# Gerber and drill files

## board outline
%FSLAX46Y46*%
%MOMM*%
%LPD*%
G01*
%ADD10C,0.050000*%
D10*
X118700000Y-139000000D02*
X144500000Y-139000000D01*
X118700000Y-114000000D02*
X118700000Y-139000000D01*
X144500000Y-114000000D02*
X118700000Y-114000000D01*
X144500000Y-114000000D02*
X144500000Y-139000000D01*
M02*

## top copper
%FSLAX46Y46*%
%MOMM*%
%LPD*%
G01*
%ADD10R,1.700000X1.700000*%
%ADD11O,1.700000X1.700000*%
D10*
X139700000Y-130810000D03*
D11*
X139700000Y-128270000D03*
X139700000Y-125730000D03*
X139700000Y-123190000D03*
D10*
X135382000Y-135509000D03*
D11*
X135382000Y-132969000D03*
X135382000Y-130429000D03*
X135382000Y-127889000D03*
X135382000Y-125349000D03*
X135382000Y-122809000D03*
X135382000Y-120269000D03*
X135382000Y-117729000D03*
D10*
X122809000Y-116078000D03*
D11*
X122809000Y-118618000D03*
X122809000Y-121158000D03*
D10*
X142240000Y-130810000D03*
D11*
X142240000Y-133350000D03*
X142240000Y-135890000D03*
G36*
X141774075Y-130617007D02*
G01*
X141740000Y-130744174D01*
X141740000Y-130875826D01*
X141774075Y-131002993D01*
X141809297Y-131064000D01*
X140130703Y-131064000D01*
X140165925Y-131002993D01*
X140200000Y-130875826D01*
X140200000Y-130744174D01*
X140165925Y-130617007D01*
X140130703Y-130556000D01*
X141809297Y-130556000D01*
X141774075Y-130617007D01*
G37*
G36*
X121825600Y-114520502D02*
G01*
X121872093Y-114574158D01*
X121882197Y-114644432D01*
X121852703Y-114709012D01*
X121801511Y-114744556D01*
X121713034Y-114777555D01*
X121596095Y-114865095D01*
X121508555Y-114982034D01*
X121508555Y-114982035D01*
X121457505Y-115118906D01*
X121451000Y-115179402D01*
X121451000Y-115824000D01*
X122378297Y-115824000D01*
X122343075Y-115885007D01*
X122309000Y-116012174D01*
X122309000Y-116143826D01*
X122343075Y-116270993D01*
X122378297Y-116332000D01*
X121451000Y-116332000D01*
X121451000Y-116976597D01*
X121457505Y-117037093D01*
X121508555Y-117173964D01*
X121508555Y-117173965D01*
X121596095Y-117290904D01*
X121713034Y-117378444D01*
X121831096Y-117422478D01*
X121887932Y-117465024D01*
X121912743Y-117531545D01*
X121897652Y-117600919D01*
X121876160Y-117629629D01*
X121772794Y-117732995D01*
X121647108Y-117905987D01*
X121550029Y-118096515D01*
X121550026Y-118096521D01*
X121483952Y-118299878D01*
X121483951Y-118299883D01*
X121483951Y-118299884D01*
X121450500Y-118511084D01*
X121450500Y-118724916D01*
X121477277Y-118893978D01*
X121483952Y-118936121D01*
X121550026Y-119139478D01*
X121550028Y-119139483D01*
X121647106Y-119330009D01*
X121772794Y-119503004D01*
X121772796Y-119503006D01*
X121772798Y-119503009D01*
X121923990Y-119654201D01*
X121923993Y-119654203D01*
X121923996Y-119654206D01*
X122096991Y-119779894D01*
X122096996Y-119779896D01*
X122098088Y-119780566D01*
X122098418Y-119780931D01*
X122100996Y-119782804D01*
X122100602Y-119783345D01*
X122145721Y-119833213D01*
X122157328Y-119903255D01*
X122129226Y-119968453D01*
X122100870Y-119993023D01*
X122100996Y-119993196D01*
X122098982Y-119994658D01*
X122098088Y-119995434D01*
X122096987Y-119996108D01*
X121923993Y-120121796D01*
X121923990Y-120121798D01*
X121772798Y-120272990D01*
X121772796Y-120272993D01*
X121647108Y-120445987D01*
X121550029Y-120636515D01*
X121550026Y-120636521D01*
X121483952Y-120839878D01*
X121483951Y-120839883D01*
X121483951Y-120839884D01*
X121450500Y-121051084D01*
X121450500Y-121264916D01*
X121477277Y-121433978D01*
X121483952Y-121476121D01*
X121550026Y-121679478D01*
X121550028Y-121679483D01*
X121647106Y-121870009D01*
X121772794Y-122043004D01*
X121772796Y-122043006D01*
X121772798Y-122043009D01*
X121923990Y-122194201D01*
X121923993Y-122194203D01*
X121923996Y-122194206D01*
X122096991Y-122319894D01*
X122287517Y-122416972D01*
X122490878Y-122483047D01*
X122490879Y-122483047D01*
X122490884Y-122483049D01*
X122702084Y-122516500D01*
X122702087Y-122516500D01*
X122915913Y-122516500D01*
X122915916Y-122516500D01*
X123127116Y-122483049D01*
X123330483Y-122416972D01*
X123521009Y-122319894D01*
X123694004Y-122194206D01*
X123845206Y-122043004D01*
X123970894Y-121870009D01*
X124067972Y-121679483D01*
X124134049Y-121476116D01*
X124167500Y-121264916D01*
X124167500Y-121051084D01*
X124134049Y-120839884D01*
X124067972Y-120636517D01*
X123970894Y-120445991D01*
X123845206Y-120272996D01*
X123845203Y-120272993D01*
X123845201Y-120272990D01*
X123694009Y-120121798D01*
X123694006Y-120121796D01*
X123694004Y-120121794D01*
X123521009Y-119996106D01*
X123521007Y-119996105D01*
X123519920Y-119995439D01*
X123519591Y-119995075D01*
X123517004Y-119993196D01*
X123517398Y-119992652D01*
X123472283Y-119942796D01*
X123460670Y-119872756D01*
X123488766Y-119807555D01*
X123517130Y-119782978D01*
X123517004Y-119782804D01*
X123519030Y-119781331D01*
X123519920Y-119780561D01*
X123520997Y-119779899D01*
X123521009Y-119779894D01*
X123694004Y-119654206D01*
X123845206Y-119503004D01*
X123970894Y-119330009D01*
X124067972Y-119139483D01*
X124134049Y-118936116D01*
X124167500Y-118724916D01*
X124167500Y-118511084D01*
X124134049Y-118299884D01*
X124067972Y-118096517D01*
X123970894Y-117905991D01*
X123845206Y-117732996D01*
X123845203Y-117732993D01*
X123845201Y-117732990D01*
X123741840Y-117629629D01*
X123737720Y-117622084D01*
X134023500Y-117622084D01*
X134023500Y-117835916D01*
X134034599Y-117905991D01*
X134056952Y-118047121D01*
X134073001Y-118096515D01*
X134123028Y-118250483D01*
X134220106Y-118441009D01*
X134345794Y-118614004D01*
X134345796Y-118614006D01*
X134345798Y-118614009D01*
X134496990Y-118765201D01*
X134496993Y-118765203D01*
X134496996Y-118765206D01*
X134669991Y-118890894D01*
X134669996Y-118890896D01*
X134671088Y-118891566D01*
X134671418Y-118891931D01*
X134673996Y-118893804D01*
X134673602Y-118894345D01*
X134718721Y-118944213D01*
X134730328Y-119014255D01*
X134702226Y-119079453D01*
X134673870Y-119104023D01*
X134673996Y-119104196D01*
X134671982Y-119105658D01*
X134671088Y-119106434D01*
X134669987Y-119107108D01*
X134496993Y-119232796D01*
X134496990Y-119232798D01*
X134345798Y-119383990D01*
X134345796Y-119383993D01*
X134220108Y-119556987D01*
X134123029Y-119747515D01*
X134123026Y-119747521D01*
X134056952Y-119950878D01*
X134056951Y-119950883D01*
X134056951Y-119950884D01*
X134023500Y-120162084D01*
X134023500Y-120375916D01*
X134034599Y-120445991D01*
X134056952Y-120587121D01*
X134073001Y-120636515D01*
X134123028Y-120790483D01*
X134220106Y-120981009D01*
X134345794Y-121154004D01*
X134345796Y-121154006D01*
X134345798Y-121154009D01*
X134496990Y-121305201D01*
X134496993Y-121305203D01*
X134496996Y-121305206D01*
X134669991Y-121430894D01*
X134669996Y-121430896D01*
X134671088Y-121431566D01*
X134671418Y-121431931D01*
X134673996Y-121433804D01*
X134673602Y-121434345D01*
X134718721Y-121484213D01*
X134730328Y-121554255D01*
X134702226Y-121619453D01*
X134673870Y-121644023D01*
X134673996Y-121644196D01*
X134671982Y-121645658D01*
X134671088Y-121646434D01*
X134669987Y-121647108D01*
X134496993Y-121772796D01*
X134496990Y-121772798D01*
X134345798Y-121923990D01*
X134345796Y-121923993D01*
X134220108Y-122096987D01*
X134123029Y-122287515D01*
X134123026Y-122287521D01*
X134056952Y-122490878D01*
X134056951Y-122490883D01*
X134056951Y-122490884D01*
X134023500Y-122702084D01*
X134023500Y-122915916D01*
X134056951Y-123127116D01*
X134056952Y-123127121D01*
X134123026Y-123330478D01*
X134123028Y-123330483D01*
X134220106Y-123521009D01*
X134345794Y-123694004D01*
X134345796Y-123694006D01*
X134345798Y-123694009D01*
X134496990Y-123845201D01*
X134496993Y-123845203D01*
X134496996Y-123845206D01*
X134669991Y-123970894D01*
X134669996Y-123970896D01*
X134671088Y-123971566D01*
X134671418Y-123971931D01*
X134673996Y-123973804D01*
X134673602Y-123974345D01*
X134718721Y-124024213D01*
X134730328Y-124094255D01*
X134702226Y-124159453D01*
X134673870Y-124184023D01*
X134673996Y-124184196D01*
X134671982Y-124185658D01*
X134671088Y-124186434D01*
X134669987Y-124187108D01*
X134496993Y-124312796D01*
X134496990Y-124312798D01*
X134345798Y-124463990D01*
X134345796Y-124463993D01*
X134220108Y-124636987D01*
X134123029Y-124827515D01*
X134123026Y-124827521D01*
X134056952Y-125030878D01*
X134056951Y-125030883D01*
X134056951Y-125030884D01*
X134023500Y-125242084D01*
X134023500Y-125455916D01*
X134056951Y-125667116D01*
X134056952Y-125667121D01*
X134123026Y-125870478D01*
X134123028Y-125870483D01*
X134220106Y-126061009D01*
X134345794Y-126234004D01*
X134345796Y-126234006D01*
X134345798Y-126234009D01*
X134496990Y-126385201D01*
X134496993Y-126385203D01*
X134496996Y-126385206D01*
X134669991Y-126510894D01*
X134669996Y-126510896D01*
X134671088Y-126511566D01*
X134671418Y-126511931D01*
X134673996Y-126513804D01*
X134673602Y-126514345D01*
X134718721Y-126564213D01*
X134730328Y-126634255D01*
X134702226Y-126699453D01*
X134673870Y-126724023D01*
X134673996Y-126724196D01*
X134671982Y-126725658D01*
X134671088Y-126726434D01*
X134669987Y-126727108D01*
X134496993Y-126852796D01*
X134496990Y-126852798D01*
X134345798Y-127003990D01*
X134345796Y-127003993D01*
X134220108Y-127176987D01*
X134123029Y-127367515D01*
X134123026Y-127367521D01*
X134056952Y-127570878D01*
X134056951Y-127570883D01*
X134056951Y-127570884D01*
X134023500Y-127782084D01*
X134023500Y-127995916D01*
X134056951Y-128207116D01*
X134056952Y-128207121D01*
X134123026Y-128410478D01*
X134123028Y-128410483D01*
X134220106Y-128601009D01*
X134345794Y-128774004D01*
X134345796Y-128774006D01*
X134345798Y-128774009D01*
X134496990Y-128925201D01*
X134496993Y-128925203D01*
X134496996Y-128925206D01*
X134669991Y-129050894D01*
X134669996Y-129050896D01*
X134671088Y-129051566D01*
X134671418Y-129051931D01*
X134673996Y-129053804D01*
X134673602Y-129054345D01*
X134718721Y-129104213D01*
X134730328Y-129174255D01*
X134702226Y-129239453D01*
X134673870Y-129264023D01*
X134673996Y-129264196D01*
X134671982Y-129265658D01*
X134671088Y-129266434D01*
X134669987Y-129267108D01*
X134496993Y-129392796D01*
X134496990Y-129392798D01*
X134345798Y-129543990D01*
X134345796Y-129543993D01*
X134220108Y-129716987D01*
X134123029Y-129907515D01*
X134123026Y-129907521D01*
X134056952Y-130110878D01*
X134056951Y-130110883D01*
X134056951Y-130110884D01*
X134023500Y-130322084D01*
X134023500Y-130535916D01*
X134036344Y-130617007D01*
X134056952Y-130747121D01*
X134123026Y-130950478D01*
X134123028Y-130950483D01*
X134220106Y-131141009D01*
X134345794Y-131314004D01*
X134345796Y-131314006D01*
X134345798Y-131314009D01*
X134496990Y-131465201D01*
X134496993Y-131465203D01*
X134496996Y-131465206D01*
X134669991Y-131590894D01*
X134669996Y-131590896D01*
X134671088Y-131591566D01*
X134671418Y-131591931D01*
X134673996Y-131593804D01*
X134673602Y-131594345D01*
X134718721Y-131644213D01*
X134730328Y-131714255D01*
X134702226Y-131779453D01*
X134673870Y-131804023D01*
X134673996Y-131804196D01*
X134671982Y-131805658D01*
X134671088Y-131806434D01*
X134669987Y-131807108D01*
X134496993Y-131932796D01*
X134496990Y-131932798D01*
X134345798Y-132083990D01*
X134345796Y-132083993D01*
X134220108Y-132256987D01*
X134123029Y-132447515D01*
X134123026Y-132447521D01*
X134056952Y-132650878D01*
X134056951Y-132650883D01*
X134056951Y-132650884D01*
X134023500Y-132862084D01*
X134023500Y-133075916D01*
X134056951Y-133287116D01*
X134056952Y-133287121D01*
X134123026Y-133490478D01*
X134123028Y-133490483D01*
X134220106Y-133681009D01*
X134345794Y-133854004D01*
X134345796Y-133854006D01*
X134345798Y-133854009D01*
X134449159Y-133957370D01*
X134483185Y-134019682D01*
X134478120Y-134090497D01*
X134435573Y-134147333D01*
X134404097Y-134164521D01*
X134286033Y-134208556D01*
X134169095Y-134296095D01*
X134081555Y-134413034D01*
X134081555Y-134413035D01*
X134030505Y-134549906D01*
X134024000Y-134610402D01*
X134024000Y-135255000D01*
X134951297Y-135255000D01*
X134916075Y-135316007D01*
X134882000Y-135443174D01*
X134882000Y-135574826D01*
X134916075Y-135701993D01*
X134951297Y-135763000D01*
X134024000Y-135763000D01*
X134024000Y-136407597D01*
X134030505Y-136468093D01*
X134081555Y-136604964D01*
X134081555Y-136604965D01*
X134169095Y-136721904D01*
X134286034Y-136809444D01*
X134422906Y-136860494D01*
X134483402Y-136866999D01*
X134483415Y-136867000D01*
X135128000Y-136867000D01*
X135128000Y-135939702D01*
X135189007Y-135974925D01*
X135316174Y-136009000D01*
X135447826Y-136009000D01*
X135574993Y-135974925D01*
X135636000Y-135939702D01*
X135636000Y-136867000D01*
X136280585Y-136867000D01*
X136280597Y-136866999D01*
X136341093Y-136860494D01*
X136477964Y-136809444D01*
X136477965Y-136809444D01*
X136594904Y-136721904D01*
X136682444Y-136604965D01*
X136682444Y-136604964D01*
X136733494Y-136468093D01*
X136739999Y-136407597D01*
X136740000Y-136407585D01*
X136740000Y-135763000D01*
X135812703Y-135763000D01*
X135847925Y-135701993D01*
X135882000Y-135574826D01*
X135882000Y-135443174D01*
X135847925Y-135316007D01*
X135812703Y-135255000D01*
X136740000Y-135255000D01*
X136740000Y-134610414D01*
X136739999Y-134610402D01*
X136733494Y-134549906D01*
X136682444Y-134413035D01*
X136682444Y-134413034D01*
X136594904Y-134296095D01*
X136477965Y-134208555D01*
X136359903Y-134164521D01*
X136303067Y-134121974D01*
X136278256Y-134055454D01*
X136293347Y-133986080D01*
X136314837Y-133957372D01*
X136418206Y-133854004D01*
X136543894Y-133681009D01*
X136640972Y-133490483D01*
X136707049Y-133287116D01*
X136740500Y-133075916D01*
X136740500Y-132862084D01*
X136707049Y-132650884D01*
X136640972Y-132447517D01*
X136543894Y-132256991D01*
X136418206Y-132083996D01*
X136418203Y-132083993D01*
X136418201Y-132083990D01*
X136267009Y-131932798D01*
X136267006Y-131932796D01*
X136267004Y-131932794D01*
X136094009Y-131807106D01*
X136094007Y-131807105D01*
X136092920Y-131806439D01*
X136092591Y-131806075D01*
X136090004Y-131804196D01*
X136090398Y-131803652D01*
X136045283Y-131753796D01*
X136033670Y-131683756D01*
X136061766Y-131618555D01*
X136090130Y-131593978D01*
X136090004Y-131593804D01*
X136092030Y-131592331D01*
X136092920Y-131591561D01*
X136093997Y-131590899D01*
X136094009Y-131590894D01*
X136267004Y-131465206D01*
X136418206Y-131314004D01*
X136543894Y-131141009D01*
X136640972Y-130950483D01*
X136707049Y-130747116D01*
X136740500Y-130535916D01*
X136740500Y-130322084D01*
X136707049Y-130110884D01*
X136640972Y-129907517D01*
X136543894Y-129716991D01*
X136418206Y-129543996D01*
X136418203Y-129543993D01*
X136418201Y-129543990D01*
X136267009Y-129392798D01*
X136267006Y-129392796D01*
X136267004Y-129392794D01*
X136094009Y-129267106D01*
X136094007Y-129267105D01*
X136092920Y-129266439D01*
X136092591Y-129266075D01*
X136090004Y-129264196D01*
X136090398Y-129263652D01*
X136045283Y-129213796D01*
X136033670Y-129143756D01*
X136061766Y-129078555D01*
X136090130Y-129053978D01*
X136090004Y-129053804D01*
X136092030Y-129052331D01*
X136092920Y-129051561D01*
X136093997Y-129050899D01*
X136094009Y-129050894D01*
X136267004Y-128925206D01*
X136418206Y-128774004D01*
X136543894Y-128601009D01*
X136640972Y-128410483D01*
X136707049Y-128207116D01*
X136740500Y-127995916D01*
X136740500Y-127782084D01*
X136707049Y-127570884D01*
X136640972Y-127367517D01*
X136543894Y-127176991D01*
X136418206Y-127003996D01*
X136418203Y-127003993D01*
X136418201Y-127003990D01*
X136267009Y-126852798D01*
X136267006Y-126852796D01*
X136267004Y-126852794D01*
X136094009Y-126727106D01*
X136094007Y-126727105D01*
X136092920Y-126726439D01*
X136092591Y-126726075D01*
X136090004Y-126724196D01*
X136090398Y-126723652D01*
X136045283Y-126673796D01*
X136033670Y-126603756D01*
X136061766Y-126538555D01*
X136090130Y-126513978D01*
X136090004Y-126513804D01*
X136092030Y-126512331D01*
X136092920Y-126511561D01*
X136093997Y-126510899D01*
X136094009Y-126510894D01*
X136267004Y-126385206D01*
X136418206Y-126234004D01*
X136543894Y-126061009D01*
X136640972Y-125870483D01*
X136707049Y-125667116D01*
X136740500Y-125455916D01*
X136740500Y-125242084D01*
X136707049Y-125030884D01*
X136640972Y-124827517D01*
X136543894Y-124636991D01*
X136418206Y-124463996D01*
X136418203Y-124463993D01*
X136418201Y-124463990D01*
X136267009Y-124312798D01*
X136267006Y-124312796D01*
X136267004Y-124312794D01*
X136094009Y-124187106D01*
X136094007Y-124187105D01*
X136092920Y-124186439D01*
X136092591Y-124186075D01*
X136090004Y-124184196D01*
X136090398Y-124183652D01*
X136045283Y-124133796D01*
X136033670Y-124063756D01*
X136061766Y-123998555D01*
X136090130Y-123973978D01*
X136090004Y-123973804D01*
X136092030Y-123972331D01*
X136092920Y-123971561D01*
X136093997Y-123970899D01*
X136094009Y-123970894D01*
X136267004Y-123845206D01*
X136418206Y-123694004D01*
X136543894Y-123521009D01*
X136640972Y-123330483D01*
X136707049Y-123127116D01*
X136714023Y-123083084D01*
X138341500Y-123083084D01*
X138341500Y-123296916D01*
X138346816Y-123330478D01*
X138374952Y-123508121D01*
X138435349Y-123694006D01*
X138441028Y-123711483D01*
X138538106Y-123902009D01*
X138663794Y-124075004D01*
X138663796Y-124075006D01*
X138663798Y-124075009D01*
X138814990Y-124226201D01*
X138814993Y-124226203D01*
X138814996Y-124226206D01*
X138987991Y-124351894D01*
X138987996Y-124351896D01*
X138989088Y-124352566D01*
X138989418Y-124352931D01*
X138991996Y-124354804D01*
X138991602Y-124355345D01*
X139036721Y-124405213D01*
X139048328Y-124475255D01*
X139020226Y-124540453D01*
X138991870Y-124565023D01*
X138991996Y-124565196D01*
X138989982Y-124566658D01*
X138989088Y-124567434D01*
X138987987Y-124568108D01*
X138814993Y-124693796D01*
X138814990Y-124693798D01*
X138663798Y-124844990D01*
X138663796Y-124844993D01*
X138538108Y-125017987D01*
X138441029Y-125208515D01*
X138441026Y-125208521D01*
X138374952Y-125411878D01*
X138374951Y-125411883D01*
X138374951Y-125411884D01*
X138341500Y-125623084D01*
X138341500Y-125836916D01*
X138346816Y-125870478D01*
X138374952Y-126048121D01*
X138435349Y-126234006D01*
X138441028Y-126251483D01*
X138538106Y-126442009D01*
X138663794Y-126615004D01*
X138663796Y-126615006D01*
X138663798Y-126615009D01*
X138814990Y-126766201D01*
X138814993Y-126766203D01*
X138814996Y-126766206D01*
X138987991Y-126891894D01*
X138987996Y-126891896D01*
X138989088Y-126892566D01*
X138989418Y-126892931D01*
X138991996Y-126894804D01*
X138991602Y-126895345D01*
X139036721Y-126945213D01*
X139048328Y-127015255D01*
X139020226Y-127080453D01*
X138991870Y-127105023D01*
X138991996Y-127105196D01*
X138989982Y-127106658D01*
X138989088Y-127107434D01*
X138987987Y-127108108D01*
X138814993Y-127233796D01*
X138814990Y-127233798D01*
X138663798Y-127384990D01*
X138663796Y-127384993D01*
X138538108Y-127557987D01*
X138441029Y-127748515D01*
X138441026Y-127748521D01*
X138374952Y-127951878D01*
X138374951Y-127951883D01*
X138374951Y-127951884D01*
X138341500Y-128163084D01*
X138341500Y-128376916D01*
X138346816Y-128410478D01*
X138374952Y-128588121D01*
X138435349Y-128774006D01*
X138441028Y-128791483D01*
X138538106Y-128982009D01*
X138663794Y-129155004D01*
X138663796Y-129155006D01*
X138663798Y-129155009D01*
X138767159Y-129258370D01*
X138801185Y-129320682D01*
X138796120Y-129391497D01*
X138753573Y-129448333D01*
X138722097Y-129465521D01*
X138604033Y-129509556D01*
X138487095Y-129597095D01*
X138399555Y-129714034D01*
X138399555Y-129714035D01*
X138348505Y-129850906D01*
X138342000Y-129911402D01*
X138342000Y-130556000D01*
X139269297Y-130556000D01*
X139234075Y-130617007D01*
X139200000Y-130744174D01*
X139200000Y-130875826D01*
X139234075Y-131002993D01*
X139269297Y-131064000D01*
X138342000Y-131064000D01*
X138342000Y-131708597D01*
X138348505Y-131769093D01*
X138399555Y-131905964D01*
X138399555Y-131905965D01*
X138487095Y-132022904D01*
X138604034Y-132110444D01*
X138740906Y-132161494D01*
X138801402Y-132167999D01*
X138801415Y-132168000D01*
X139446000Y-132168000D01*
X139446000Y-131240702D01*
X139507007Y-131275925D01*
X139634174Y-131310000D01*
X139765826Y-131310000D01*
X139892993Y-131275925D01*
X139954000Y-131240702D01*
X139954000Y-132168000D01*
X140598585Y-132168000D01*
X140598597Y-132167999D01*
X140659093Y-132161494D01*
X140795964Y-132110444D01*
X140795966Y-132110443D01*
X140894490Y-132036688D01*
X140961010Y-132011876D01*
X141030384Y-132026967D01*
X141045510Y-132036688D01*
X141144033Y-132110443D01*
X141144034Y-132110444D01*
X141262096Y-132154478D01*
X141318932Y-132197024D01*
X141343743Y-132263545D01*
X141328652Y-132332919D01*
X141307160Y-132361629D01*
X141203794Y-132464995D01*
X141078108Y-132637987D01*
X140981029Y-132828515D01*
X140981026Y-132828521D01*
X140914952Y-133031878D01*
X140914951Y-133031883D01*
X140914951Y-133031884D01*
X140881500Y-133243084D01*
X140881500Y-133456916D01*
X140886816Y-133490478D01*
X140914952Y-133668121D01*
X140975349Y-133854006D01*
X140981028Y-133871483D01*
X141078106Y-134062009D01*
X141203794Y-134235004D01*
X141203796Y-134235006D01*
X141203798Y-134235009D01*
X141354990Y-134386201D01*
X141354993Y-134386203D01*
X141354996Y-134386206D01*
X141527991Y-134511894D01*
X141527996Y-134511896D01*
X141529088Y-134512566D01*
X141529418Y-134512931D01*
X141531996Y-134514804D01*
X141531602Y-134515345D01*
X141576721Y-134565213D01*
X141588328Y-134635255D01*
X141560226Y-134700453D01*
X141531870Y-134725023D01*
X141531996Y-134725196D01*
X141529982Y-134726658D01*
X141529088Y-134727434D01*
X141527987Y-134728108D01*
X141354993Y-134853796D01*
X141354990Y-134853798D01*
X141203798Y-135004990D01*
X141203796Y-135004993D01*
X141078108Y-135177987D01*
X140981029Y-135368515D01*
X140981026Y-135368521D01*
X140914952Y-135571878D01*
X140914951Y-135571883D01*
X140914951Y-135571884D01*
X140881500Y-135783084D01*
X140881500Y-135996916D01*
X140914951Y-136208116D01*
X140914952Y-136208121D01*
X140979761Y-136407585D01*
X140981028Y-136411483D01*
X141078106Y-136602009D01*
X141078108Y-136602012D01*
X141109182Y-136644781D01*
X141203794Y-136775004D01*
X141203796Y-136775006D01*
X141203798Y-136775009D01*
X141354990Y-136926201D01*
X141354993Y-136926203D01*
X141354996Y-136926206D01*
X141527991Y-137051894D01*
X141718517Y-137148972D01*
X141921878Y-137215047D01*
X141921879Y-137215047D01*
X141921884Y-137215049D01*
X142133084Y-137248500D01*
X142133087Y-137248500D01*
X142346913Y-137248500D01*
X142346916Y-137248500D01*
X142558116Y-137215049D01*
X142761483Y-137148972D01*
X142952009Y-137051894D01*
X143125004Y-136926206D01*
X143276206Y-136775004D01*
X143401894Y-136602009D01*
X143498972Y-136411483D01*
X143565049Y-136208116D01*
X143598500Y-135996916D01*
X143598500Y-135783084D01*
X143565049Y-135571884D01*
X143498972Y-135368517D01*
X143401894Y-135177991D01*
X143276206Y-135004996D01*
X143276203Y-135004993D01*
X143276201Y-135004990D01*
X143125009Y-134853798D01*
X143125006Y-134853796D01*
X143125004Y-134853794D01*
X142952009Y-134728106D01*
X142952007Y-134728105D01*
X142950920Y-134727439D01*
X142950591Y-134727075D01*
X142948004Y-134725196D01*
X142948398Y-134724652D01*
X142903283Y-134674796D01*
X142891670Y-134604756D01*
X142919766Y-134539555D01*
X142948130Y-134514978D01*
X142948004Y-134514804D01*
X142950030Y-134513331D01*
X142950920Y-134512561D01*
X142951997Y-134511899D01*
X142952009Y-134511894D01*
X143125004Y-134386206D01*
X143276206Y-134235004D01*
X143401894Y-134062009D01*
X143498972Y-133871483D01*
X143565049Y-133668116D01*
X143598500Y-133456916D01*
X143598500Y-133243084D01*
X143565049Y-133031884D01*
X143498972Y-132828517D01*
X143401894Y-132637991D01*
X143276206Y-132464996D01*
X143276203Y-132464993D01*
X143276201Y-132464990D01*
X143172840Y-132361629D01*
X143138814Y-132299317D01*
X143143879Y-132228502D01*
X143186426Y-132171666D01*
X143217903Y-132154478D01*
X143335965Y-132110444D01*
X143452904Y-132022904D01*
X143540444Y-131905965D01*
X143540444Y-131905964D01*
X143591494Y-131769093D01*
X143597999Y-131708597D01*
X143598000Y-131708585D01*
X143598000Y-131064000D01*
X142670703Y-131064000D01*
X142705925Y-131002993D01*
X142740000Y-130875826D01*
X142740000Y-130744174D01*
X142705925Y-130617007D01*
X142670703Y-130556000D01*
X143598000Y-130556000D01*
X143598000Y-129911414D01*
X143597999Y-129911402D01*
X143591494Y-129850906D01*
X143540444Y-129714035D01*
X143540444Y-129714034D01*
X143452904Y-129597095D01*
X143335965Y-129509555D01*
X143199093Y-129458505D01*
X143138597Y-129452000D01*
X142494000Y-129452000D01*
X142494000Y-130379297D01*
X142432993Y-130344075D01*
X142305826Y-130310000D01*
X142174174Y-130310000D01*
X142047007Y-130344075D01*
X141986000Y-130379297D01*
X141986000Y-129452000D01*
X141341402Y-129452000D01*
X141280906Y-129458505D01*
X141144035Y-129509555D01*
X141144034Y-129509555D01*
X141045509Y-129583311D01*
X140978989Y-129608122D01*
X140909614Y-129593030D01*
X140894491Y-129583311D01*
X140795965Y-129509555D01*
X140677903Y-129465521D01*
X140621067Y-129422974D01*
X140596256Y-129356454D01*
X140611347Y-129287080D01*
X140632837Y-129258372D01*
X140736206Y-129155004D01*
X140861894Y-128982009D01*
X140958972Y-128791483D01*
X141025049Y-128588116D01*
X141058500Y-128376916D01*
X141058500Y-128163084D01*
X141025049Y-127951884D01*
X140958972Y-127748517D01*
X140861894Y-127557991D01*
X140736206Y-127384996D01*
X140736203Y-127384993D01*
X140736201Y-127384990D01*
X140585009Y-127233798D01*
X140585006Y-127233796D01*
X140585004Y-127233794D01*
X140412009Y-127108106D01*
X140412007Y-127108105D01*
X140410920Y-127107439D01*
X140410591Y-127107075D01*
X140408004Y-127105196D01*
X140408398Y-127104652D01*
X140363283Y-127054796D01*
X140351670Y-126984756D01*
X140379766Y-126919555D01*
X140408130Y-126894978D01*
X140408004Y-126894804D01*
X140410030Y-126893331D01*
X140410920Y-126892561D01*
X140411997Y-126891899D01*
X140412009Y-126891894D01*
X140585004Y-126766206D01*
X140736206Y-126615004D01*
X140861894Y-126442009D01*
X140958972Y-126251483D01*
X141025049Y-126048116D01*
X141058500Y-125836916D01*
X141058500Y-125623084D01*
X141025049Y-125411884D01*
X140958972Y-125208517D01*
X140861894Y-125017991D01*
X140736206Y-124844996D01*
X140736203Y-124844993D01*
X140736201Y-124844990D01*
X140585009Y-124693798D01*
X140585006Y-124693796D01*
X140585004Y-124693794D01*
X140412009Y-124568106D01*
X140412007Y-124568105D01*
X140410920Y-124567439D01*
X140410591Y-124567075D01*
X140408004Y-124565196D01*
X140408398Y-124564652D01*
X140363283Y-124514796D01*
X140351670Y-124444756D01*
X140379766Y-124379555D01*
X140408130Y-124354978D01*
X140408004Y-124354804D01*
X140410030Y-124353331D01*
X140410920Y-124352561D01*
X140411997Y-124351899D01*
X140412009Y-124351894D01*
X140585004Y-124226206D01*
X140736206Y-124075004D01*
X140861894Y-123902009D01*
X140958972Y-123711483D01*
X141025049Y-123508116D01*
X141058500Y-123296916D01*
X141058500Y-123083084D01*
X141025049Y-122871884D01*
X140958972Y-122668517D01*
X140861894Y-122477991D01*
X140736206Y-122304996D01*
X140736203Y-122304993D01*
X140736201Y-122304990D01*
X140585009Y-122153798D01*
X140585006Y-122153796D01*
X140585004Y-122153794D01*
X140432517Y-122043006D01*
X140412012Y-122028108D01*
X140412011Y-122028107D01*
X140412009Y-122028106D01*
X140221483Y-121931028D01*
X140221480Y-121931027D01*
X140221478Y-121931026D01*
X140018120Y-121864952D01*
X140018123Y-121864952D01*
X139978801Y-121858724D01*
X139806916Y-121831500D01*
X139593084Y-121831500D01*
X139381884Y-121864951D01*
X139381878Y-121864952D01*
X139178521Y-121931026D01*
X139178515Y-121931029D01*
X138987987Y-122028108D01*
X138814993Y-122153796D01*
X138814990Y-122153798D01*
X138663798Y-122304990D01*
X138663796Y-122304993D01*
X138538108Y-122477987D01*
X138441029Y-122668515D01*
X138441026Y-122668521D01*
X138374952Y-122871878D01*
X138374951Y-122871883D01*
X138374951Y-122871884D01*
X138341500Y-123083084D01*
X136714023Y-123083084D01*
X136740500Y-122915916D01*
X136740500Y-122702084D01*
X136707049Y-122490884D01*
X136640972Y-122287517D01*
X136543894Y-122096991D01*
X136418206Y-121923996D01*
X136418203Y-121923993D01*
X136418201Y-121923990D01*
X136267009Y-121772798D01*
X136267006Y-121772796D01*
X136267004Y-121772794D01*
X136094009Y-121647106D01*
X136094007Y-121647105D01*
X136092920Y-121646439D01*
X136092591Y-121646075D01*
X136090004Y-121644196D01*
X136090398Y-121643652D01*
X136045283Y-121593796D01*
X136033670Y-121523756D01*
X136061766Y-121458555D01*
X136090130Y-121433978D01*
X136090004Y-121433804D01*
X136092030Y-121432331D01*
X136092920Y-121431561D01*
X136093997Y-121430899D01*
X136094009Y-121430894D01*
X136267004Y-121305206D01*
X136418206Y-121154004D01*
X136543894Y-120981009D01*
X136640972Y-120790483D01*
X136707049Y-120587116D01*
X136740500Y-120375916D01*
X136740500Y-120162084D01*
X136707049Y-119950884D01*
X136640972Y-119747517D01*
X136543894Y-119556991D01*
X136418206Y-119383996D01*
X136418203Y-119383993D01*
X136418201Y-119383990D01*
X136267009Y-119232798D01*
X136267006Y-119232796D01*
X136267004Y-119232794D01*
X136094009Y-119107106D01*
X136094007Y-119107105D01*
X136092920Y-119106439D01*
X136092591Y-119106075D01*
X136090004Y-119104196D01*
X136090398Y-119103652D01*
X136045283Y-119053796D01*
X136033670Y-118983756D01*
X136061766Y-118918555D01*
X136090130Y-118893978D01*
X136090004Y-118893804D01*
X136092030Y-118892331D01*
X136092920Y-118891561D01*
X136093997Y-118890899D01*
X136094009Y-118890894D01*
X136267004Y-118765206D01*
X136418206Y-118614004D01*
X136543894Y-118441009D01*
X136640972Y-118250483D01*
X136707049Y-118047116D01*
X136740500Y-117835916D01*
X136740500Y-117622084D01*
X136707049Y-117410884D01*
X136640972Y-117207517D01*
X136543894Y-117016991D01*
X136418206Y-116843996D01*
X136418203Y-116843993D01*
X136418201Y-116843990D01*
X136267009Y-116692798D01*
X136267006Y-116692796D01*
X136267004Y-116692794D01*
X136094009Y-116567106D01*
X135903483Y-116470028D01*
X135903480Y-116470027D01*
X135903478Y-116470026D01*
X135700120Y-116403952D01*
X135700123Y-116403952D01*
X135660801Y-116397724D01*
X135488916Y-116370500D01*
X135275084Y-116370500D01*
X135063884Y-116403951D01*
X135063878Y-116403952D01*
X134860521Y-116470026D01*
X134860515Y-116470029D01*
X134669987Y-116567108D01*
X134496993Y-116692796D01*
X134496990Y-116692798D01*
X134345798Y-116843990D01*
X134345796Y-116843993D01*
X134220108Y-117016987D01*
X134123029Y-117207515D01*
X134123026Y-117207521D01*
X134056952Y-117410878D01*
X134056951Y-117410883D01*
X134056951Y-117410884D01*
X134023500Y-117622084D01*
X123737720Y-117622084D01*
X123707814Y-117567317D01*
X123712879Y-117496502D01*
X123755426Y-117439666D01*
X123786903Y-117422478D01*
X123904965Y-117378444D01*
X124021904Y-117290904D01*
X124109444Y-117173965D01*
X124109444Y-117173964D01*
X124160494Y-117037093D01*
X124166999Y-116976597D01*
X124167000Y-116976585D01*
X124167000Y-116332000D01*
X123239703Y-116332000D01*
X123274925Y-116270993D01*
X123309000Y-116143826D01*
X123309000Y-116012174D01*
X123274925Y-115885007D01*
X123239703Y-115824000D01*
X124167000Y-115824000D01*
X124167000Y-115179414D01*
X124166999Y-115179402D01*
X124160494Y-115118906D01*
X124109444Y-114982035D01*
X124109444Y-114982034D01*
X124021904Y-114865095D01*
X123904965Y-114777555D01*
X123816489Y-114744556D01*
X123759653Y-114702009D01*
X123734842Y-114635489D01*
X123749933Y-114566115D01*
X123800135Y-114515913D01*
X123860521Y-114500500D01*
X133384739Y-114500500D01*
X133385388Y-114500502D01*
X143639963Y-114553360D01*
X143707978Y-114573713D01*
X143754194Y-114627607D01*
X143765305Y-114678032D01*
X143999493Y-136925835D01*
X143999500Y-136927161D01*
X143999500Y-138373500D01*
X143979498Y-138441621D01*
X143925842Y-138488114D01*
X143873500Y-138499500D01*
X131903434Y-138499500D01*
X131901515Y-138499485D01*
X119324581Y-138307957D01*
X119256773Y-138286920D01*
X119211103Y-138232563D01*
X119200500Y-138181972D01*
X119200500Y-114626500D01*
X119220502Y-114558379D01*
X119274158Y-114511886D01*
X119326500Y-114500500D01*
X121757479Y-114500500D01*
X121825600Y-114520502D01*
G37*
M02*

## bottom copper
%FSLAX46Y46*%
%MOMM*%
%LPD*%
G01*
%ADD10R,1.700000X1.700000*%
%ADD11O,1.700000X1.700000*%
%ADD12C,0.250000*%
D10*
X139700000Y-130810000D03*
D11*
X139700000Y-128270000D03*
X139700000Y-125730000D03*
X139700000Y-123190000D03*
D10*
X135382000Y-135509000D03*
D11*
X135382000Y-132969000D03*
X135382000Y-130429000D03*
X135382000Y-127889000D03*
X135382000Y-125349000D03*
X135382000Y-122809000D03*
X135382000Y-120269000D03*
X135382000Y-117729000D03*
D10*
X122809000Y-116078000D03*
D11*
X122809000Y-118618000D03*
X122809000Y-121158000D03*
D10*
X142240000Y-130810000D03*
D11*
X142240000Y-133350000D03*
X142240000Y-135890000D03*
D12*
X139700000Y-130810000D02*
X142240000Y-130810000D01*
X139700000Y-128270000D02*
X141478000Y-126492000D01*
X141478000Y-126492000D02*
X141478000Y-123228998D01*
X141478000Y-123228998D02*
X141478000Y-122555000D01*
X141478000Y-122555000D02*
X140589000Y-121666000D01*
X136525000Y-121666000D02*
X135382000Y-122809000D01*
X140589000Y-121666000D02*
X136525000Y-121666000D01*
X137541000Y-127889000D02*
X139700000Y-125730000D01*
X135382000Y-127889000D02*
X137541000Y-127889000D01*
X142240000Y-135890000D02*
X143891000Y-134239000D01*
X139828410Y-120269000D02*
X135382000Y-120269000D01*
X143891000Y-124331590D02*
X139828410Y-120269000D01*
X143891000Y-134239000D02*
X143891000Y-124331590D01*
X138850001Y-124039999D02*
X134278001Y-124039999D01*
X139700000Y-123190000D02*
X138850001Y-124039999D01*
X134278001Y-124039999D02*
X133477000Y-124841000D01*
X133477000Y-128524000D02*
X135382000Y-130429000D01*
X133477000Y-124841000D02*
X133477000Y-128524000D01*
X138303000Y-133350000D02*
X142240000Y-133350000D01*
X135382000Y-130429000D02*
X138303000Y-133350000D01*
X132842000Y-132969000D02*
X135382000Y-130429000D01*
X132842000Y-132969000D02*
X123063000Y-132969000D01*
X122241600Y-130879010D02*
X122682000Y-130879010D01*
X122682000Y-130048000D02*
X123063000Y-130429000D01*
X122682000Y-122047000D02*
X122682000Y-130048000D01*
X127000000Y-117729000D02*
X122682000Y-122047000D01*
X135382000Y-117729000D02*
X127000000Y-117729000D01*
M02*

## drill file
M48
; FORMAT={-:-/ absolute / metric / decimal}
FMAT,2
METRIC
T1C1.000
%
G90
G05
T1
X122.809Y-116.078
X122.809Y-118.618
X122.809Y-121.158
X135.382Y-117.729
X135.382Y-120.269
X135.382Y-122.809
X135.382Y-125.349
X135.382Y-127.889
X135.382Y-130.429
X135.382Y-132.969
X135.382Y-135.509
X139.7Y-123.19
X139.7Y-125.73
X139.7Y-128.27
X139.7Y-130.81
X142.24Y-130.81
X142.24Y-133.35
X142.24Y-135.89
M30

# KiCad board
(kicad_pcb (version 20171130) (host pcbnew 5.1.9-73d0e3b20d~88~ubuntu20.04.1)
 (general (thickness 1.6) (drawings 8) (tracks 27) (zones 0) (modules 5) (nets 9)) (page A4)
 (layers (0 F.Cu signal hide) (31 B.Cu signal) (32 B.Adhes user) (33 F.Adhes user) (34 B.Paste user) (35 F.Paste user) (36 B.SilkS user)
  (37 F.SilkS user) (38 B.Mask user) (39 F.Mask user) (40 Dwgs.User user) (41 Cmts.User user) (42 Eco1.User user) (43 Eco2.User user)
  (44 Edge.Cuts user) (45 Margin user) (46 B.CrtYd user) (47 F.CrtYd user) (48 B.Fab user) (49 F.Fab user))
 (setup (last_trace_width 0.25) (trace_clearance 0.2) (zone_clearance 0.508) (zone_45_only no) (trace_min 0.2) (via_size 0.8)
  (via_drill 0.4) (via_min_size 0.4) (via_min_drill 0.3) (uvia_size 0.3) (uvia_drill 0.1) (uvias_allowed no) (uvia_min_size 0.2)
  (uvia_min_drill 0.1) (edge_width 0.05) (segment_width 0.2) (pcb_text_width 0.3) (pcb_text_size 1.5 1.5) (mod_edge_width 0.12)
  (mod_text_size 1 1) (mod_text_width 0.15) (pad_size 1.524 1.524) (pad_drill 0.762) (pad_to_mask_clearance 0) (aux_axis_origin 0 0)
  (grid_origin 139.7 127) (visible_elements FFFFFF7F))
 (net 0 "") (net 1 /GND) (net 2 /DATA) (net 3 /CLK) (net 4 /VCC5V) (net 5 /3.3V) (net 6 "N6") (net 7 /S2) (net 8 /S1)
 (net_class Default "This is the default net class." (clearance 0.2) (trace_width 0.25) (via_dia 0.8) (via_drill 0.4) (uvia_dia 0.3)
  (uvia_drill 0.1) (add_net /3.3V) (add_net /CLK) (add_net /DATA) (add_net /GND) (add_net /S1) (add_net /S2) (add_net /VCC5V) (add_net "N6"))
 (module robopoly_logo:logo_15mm (layer F.Cu) (at 122.047 131.445 270)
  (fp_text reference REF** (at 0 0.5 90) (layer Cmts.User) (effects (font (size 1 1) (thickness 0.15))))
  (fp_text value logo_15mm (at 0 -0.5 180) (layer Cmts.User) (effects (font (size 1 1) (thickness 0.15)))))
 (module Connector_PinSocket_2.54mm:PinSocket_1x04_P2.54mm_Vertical (layer B.Cu) (at 139.7 130.81)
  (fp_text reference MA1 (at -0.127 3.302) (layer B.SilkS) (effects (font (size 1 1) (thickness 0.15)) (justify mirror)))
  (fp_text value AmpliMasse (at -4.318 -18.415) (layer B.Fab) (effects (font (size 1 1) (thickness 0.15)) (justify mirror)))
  (pad 1 thru_hole rect (at 0 0) (size 1.7 1.7) (drill 1) (layers *.Cu *.Mask) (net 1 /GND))
  (pad 2 thru_hole oval (at 0 -2.54) (size 1.7 1.7) (drill 1) (layers *.Cu *.Mask) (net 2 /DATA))
  (pad 3 thru_hole oval (at 0 -5.08) (size 1.7 1.7) (drill 1) (layers *.Cu *.Mask) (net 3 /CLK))
  (pad 4 thru_hole oval (at 0 -7.62) (size 1.7 1.7) (drill 1) (layers *.Cu *.Mask) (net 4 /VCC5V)))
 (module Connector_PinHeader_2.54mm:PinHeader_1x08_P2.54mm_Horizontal (layer F.Cu) (at 135.382 135.509 180)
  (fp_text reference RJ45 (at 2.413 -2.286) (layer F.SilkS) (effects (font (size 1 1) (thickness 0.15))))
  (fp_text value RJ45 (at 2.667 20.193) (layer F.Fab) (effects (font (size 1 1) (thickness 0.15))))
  (pad 1 thru_hole rect (at 0 0 180) (size 1.7 1.7) (drill 1) (layers *.Cu *.Mask) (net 1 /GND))
  (pad 2 thru_hole oval (at 0 2.54 180) (size 1.7 1.7) (drill 1) (layers *.Cu *.Mask) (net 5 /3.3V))
  (pad 3 thru_hole oval (at 0 5.08 180) (size 1.7 1.7) (drill 1) (layers *.Cu *.Mask) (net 4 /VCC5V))
  (pad 4 thru_hole oval (at 0 7.62 180) (size 1.7 1.7) (drill 1) (layers *.Cu *.Mask) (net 3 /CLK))
  (pad 5 thru_hole oval (at 0 10.16 180) (size 1.7 1.7) (drill 1) (layers *.Cu *.Mask) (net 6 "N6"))
  (pad 6 thru_hole oval (at 0 12.7 180) (size 1.7 1.7) (drill 1) (layers *.Cu *.Mask) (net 2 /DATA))
  (pad 7 thru_hole oval (at 0 15.24 180) (size 1.7 1.7) (drill 1) (layers *.Cu *.Mask) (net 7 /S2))
  (pad 8 thru_hole oval (at 0 17.78 180) (size 1.7 1.7) (drill 1) (layers *.Cu *.Mask) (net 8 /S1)))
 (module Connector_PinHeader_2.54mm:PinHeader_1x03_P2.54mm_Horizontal (layer B.Cu) (at 122.809 116.078 180)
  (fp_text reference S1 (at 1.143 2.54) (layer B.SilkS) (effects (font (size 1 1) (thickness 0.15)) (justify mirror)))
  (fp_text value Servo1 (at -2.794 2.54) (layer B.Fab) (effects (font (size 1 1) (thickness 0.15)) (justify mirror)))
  (pad 1 thru_hole rect (at 0 0 180) (size 1.7 1.7) (drill 1) (layers *.Cu *.Mask) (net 1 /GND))
  (pad 2 thru_hole oval (at 0 -2.54 180) (size 1.7 1.7) (drill 1) (layers *.Cu *.Mask) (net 4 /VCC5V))
  (pad 3 thru_hole oval (at 0 -5.08 180) (size 1.7 1.7) (drill 1) (layers *.Cu *.Mask) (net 8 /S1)))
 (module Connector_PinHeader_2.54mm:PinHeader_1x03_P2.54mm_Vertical (layer F.Cu) (at 142.24 130.81)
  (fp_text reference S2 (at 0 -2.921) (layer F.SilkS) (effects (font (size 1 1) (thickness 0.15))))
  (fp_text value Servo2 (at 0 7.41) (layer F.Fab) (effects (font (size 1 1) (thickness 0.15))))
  (pad 1 thru_hole rect (at 0 0) (size 1.7 1.7) (drill 1) (layers *.Cu *.Mask) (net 1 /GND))
  (pad 2 thru_hole oval (at 0 2.54) (size 1.7 1.7) (drill 1) (layers *.Cu *.Mask) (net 4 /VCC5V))
  (pad 3 thru_hole oval (at 0 5.08) (size 1.7 1.7) (drill 1) (layers *.Cu *.Mask) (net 7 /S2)))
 (gr_line (start 118.7 139) (end 144.5 139) (layer Edge.Cuts) (width 0.05))
 (gr_line (start 118.7 114) (end 118.7 139) (layer Edge.Cuts) (width 0.05))
 (gr_line (start 144.5 114) (end 118.7 114) (layer Edge.Cuts) (width 0.05))
 (gr_line (start 144.5 114) (end 144.5 139) (layer Edge.Cuts) (width 0.05))
 (segment (start 139.7 130.81) (end 142.24 130.81) (width 0.25) (layer B.Cu) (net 1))
 (segment (start 139.7 128.27) (end 141.478 126.492) (width 0.25) (layer B.Cu) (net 2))
 (segment (start 141.478 126.492) (end 141.478 123.228998) (width 0.25) (layer B.Cu) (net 2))
 (segment (start 141.478 123.228998) (end 141.478 122.555) (width 0.25) (layer B.Cu) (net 2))
 (segment (start 141.478 122.555) (end 140.589 121.666) (width 0.25) (layer B.Cu) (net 2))
 (segment (start 136.525 121.666) (end 135.382 122.809) (width 0.25) (layer B.Cu) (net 2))
 (segment (start 140.589 121.666) (end 136.525 121.666) (width 0.25) (layer B.Cu) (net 2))
 (segment (start 137.541 127.889) (end 139.7 125.73) (width 0.25) (layer B.Cu) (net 3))
 (segment (start 135.382 127.889) (end 137.541 127.889) (width 0.25) (layer B.Cu) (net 3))
 (segment (start 142.24 135.89) (end 143.891 134.239) (width 0.25) (layer B.Cu) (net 7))
 (segment (start 139.82841 120.269) (end 135.382 120.269) (width 0.25) (layer B.Cu) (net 7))
 (segment (start 143.891 124.33159) (end 139.82841 120.269) (width 0.25) (layer B.Cu) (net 7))
 (segment (start 143.891 134.239) (end 143.891 124.33159) (width 0.25) (layer B.Cu) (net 7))
 (segment (start 138.850001 124.039999) (end 134.278001 124.039999) (width 0.25) (layer B.Cu) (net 4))
 (segment (start 139.7 123.19) (end 138.850001 124.039999) (width 0.25) (layer B.Cu) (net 4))
 (segment (start 134.278001 124.039999) (end 133.477 124.841) (width 0.25) (layer B.Cu) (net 4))
 (segment (start 133.477 128.524) (end 135.382 130.429) (width 0.25) (layer B.Cu) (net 4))
 (segment (start 133.477 124.841) (end 133.477 128.524) (width 0.25) (layer B.Cu) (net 4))
 (segment (start 138.303 133.35) (end 142.24 133.35) (width 0.25) (layer B.Cu) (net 4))
 (segment (start 135.382 130.429) (end 138.303 133.35) (width 0.25) (layer B.Cu) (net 4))
 (segment (start 132.842 132.969) (end 135.382 130.429) (width 0.25) (layer B.Cu) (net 4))
 (segment (start 132.842 132.969) (end 123.063 132.969) (width 0.25) (layer B.Cu) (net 4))
 (segment (start 122.2416 130.87901) (end 122.682 130.87901) (width 0.25) (layer B.Cu) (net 8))
 (segment (start 122.682 130.048) (end 123.063 130.429) (width 0.25) (layer B.Cu) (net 8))
 (segment (start 122.682 122.047) (end 122.682 130.048) (width 0.25) (layer B.Cu) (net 8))
 (segment (start 127 117.729) (end 122.682 122.047) (width 0.25) (layer B.Cu) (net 8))
 (segment (start 135.382 117.729) (end 127 117.729) (width 0.25) (layer B.Cu) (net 8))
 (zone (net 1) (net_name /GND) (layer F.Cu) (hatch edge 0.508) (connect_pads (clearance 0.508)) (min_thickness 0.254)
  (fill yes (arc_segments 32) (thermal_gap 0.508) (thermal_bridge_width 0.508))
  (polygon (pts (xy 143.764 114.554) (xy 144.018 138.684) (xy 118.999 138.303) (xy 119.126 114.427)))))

